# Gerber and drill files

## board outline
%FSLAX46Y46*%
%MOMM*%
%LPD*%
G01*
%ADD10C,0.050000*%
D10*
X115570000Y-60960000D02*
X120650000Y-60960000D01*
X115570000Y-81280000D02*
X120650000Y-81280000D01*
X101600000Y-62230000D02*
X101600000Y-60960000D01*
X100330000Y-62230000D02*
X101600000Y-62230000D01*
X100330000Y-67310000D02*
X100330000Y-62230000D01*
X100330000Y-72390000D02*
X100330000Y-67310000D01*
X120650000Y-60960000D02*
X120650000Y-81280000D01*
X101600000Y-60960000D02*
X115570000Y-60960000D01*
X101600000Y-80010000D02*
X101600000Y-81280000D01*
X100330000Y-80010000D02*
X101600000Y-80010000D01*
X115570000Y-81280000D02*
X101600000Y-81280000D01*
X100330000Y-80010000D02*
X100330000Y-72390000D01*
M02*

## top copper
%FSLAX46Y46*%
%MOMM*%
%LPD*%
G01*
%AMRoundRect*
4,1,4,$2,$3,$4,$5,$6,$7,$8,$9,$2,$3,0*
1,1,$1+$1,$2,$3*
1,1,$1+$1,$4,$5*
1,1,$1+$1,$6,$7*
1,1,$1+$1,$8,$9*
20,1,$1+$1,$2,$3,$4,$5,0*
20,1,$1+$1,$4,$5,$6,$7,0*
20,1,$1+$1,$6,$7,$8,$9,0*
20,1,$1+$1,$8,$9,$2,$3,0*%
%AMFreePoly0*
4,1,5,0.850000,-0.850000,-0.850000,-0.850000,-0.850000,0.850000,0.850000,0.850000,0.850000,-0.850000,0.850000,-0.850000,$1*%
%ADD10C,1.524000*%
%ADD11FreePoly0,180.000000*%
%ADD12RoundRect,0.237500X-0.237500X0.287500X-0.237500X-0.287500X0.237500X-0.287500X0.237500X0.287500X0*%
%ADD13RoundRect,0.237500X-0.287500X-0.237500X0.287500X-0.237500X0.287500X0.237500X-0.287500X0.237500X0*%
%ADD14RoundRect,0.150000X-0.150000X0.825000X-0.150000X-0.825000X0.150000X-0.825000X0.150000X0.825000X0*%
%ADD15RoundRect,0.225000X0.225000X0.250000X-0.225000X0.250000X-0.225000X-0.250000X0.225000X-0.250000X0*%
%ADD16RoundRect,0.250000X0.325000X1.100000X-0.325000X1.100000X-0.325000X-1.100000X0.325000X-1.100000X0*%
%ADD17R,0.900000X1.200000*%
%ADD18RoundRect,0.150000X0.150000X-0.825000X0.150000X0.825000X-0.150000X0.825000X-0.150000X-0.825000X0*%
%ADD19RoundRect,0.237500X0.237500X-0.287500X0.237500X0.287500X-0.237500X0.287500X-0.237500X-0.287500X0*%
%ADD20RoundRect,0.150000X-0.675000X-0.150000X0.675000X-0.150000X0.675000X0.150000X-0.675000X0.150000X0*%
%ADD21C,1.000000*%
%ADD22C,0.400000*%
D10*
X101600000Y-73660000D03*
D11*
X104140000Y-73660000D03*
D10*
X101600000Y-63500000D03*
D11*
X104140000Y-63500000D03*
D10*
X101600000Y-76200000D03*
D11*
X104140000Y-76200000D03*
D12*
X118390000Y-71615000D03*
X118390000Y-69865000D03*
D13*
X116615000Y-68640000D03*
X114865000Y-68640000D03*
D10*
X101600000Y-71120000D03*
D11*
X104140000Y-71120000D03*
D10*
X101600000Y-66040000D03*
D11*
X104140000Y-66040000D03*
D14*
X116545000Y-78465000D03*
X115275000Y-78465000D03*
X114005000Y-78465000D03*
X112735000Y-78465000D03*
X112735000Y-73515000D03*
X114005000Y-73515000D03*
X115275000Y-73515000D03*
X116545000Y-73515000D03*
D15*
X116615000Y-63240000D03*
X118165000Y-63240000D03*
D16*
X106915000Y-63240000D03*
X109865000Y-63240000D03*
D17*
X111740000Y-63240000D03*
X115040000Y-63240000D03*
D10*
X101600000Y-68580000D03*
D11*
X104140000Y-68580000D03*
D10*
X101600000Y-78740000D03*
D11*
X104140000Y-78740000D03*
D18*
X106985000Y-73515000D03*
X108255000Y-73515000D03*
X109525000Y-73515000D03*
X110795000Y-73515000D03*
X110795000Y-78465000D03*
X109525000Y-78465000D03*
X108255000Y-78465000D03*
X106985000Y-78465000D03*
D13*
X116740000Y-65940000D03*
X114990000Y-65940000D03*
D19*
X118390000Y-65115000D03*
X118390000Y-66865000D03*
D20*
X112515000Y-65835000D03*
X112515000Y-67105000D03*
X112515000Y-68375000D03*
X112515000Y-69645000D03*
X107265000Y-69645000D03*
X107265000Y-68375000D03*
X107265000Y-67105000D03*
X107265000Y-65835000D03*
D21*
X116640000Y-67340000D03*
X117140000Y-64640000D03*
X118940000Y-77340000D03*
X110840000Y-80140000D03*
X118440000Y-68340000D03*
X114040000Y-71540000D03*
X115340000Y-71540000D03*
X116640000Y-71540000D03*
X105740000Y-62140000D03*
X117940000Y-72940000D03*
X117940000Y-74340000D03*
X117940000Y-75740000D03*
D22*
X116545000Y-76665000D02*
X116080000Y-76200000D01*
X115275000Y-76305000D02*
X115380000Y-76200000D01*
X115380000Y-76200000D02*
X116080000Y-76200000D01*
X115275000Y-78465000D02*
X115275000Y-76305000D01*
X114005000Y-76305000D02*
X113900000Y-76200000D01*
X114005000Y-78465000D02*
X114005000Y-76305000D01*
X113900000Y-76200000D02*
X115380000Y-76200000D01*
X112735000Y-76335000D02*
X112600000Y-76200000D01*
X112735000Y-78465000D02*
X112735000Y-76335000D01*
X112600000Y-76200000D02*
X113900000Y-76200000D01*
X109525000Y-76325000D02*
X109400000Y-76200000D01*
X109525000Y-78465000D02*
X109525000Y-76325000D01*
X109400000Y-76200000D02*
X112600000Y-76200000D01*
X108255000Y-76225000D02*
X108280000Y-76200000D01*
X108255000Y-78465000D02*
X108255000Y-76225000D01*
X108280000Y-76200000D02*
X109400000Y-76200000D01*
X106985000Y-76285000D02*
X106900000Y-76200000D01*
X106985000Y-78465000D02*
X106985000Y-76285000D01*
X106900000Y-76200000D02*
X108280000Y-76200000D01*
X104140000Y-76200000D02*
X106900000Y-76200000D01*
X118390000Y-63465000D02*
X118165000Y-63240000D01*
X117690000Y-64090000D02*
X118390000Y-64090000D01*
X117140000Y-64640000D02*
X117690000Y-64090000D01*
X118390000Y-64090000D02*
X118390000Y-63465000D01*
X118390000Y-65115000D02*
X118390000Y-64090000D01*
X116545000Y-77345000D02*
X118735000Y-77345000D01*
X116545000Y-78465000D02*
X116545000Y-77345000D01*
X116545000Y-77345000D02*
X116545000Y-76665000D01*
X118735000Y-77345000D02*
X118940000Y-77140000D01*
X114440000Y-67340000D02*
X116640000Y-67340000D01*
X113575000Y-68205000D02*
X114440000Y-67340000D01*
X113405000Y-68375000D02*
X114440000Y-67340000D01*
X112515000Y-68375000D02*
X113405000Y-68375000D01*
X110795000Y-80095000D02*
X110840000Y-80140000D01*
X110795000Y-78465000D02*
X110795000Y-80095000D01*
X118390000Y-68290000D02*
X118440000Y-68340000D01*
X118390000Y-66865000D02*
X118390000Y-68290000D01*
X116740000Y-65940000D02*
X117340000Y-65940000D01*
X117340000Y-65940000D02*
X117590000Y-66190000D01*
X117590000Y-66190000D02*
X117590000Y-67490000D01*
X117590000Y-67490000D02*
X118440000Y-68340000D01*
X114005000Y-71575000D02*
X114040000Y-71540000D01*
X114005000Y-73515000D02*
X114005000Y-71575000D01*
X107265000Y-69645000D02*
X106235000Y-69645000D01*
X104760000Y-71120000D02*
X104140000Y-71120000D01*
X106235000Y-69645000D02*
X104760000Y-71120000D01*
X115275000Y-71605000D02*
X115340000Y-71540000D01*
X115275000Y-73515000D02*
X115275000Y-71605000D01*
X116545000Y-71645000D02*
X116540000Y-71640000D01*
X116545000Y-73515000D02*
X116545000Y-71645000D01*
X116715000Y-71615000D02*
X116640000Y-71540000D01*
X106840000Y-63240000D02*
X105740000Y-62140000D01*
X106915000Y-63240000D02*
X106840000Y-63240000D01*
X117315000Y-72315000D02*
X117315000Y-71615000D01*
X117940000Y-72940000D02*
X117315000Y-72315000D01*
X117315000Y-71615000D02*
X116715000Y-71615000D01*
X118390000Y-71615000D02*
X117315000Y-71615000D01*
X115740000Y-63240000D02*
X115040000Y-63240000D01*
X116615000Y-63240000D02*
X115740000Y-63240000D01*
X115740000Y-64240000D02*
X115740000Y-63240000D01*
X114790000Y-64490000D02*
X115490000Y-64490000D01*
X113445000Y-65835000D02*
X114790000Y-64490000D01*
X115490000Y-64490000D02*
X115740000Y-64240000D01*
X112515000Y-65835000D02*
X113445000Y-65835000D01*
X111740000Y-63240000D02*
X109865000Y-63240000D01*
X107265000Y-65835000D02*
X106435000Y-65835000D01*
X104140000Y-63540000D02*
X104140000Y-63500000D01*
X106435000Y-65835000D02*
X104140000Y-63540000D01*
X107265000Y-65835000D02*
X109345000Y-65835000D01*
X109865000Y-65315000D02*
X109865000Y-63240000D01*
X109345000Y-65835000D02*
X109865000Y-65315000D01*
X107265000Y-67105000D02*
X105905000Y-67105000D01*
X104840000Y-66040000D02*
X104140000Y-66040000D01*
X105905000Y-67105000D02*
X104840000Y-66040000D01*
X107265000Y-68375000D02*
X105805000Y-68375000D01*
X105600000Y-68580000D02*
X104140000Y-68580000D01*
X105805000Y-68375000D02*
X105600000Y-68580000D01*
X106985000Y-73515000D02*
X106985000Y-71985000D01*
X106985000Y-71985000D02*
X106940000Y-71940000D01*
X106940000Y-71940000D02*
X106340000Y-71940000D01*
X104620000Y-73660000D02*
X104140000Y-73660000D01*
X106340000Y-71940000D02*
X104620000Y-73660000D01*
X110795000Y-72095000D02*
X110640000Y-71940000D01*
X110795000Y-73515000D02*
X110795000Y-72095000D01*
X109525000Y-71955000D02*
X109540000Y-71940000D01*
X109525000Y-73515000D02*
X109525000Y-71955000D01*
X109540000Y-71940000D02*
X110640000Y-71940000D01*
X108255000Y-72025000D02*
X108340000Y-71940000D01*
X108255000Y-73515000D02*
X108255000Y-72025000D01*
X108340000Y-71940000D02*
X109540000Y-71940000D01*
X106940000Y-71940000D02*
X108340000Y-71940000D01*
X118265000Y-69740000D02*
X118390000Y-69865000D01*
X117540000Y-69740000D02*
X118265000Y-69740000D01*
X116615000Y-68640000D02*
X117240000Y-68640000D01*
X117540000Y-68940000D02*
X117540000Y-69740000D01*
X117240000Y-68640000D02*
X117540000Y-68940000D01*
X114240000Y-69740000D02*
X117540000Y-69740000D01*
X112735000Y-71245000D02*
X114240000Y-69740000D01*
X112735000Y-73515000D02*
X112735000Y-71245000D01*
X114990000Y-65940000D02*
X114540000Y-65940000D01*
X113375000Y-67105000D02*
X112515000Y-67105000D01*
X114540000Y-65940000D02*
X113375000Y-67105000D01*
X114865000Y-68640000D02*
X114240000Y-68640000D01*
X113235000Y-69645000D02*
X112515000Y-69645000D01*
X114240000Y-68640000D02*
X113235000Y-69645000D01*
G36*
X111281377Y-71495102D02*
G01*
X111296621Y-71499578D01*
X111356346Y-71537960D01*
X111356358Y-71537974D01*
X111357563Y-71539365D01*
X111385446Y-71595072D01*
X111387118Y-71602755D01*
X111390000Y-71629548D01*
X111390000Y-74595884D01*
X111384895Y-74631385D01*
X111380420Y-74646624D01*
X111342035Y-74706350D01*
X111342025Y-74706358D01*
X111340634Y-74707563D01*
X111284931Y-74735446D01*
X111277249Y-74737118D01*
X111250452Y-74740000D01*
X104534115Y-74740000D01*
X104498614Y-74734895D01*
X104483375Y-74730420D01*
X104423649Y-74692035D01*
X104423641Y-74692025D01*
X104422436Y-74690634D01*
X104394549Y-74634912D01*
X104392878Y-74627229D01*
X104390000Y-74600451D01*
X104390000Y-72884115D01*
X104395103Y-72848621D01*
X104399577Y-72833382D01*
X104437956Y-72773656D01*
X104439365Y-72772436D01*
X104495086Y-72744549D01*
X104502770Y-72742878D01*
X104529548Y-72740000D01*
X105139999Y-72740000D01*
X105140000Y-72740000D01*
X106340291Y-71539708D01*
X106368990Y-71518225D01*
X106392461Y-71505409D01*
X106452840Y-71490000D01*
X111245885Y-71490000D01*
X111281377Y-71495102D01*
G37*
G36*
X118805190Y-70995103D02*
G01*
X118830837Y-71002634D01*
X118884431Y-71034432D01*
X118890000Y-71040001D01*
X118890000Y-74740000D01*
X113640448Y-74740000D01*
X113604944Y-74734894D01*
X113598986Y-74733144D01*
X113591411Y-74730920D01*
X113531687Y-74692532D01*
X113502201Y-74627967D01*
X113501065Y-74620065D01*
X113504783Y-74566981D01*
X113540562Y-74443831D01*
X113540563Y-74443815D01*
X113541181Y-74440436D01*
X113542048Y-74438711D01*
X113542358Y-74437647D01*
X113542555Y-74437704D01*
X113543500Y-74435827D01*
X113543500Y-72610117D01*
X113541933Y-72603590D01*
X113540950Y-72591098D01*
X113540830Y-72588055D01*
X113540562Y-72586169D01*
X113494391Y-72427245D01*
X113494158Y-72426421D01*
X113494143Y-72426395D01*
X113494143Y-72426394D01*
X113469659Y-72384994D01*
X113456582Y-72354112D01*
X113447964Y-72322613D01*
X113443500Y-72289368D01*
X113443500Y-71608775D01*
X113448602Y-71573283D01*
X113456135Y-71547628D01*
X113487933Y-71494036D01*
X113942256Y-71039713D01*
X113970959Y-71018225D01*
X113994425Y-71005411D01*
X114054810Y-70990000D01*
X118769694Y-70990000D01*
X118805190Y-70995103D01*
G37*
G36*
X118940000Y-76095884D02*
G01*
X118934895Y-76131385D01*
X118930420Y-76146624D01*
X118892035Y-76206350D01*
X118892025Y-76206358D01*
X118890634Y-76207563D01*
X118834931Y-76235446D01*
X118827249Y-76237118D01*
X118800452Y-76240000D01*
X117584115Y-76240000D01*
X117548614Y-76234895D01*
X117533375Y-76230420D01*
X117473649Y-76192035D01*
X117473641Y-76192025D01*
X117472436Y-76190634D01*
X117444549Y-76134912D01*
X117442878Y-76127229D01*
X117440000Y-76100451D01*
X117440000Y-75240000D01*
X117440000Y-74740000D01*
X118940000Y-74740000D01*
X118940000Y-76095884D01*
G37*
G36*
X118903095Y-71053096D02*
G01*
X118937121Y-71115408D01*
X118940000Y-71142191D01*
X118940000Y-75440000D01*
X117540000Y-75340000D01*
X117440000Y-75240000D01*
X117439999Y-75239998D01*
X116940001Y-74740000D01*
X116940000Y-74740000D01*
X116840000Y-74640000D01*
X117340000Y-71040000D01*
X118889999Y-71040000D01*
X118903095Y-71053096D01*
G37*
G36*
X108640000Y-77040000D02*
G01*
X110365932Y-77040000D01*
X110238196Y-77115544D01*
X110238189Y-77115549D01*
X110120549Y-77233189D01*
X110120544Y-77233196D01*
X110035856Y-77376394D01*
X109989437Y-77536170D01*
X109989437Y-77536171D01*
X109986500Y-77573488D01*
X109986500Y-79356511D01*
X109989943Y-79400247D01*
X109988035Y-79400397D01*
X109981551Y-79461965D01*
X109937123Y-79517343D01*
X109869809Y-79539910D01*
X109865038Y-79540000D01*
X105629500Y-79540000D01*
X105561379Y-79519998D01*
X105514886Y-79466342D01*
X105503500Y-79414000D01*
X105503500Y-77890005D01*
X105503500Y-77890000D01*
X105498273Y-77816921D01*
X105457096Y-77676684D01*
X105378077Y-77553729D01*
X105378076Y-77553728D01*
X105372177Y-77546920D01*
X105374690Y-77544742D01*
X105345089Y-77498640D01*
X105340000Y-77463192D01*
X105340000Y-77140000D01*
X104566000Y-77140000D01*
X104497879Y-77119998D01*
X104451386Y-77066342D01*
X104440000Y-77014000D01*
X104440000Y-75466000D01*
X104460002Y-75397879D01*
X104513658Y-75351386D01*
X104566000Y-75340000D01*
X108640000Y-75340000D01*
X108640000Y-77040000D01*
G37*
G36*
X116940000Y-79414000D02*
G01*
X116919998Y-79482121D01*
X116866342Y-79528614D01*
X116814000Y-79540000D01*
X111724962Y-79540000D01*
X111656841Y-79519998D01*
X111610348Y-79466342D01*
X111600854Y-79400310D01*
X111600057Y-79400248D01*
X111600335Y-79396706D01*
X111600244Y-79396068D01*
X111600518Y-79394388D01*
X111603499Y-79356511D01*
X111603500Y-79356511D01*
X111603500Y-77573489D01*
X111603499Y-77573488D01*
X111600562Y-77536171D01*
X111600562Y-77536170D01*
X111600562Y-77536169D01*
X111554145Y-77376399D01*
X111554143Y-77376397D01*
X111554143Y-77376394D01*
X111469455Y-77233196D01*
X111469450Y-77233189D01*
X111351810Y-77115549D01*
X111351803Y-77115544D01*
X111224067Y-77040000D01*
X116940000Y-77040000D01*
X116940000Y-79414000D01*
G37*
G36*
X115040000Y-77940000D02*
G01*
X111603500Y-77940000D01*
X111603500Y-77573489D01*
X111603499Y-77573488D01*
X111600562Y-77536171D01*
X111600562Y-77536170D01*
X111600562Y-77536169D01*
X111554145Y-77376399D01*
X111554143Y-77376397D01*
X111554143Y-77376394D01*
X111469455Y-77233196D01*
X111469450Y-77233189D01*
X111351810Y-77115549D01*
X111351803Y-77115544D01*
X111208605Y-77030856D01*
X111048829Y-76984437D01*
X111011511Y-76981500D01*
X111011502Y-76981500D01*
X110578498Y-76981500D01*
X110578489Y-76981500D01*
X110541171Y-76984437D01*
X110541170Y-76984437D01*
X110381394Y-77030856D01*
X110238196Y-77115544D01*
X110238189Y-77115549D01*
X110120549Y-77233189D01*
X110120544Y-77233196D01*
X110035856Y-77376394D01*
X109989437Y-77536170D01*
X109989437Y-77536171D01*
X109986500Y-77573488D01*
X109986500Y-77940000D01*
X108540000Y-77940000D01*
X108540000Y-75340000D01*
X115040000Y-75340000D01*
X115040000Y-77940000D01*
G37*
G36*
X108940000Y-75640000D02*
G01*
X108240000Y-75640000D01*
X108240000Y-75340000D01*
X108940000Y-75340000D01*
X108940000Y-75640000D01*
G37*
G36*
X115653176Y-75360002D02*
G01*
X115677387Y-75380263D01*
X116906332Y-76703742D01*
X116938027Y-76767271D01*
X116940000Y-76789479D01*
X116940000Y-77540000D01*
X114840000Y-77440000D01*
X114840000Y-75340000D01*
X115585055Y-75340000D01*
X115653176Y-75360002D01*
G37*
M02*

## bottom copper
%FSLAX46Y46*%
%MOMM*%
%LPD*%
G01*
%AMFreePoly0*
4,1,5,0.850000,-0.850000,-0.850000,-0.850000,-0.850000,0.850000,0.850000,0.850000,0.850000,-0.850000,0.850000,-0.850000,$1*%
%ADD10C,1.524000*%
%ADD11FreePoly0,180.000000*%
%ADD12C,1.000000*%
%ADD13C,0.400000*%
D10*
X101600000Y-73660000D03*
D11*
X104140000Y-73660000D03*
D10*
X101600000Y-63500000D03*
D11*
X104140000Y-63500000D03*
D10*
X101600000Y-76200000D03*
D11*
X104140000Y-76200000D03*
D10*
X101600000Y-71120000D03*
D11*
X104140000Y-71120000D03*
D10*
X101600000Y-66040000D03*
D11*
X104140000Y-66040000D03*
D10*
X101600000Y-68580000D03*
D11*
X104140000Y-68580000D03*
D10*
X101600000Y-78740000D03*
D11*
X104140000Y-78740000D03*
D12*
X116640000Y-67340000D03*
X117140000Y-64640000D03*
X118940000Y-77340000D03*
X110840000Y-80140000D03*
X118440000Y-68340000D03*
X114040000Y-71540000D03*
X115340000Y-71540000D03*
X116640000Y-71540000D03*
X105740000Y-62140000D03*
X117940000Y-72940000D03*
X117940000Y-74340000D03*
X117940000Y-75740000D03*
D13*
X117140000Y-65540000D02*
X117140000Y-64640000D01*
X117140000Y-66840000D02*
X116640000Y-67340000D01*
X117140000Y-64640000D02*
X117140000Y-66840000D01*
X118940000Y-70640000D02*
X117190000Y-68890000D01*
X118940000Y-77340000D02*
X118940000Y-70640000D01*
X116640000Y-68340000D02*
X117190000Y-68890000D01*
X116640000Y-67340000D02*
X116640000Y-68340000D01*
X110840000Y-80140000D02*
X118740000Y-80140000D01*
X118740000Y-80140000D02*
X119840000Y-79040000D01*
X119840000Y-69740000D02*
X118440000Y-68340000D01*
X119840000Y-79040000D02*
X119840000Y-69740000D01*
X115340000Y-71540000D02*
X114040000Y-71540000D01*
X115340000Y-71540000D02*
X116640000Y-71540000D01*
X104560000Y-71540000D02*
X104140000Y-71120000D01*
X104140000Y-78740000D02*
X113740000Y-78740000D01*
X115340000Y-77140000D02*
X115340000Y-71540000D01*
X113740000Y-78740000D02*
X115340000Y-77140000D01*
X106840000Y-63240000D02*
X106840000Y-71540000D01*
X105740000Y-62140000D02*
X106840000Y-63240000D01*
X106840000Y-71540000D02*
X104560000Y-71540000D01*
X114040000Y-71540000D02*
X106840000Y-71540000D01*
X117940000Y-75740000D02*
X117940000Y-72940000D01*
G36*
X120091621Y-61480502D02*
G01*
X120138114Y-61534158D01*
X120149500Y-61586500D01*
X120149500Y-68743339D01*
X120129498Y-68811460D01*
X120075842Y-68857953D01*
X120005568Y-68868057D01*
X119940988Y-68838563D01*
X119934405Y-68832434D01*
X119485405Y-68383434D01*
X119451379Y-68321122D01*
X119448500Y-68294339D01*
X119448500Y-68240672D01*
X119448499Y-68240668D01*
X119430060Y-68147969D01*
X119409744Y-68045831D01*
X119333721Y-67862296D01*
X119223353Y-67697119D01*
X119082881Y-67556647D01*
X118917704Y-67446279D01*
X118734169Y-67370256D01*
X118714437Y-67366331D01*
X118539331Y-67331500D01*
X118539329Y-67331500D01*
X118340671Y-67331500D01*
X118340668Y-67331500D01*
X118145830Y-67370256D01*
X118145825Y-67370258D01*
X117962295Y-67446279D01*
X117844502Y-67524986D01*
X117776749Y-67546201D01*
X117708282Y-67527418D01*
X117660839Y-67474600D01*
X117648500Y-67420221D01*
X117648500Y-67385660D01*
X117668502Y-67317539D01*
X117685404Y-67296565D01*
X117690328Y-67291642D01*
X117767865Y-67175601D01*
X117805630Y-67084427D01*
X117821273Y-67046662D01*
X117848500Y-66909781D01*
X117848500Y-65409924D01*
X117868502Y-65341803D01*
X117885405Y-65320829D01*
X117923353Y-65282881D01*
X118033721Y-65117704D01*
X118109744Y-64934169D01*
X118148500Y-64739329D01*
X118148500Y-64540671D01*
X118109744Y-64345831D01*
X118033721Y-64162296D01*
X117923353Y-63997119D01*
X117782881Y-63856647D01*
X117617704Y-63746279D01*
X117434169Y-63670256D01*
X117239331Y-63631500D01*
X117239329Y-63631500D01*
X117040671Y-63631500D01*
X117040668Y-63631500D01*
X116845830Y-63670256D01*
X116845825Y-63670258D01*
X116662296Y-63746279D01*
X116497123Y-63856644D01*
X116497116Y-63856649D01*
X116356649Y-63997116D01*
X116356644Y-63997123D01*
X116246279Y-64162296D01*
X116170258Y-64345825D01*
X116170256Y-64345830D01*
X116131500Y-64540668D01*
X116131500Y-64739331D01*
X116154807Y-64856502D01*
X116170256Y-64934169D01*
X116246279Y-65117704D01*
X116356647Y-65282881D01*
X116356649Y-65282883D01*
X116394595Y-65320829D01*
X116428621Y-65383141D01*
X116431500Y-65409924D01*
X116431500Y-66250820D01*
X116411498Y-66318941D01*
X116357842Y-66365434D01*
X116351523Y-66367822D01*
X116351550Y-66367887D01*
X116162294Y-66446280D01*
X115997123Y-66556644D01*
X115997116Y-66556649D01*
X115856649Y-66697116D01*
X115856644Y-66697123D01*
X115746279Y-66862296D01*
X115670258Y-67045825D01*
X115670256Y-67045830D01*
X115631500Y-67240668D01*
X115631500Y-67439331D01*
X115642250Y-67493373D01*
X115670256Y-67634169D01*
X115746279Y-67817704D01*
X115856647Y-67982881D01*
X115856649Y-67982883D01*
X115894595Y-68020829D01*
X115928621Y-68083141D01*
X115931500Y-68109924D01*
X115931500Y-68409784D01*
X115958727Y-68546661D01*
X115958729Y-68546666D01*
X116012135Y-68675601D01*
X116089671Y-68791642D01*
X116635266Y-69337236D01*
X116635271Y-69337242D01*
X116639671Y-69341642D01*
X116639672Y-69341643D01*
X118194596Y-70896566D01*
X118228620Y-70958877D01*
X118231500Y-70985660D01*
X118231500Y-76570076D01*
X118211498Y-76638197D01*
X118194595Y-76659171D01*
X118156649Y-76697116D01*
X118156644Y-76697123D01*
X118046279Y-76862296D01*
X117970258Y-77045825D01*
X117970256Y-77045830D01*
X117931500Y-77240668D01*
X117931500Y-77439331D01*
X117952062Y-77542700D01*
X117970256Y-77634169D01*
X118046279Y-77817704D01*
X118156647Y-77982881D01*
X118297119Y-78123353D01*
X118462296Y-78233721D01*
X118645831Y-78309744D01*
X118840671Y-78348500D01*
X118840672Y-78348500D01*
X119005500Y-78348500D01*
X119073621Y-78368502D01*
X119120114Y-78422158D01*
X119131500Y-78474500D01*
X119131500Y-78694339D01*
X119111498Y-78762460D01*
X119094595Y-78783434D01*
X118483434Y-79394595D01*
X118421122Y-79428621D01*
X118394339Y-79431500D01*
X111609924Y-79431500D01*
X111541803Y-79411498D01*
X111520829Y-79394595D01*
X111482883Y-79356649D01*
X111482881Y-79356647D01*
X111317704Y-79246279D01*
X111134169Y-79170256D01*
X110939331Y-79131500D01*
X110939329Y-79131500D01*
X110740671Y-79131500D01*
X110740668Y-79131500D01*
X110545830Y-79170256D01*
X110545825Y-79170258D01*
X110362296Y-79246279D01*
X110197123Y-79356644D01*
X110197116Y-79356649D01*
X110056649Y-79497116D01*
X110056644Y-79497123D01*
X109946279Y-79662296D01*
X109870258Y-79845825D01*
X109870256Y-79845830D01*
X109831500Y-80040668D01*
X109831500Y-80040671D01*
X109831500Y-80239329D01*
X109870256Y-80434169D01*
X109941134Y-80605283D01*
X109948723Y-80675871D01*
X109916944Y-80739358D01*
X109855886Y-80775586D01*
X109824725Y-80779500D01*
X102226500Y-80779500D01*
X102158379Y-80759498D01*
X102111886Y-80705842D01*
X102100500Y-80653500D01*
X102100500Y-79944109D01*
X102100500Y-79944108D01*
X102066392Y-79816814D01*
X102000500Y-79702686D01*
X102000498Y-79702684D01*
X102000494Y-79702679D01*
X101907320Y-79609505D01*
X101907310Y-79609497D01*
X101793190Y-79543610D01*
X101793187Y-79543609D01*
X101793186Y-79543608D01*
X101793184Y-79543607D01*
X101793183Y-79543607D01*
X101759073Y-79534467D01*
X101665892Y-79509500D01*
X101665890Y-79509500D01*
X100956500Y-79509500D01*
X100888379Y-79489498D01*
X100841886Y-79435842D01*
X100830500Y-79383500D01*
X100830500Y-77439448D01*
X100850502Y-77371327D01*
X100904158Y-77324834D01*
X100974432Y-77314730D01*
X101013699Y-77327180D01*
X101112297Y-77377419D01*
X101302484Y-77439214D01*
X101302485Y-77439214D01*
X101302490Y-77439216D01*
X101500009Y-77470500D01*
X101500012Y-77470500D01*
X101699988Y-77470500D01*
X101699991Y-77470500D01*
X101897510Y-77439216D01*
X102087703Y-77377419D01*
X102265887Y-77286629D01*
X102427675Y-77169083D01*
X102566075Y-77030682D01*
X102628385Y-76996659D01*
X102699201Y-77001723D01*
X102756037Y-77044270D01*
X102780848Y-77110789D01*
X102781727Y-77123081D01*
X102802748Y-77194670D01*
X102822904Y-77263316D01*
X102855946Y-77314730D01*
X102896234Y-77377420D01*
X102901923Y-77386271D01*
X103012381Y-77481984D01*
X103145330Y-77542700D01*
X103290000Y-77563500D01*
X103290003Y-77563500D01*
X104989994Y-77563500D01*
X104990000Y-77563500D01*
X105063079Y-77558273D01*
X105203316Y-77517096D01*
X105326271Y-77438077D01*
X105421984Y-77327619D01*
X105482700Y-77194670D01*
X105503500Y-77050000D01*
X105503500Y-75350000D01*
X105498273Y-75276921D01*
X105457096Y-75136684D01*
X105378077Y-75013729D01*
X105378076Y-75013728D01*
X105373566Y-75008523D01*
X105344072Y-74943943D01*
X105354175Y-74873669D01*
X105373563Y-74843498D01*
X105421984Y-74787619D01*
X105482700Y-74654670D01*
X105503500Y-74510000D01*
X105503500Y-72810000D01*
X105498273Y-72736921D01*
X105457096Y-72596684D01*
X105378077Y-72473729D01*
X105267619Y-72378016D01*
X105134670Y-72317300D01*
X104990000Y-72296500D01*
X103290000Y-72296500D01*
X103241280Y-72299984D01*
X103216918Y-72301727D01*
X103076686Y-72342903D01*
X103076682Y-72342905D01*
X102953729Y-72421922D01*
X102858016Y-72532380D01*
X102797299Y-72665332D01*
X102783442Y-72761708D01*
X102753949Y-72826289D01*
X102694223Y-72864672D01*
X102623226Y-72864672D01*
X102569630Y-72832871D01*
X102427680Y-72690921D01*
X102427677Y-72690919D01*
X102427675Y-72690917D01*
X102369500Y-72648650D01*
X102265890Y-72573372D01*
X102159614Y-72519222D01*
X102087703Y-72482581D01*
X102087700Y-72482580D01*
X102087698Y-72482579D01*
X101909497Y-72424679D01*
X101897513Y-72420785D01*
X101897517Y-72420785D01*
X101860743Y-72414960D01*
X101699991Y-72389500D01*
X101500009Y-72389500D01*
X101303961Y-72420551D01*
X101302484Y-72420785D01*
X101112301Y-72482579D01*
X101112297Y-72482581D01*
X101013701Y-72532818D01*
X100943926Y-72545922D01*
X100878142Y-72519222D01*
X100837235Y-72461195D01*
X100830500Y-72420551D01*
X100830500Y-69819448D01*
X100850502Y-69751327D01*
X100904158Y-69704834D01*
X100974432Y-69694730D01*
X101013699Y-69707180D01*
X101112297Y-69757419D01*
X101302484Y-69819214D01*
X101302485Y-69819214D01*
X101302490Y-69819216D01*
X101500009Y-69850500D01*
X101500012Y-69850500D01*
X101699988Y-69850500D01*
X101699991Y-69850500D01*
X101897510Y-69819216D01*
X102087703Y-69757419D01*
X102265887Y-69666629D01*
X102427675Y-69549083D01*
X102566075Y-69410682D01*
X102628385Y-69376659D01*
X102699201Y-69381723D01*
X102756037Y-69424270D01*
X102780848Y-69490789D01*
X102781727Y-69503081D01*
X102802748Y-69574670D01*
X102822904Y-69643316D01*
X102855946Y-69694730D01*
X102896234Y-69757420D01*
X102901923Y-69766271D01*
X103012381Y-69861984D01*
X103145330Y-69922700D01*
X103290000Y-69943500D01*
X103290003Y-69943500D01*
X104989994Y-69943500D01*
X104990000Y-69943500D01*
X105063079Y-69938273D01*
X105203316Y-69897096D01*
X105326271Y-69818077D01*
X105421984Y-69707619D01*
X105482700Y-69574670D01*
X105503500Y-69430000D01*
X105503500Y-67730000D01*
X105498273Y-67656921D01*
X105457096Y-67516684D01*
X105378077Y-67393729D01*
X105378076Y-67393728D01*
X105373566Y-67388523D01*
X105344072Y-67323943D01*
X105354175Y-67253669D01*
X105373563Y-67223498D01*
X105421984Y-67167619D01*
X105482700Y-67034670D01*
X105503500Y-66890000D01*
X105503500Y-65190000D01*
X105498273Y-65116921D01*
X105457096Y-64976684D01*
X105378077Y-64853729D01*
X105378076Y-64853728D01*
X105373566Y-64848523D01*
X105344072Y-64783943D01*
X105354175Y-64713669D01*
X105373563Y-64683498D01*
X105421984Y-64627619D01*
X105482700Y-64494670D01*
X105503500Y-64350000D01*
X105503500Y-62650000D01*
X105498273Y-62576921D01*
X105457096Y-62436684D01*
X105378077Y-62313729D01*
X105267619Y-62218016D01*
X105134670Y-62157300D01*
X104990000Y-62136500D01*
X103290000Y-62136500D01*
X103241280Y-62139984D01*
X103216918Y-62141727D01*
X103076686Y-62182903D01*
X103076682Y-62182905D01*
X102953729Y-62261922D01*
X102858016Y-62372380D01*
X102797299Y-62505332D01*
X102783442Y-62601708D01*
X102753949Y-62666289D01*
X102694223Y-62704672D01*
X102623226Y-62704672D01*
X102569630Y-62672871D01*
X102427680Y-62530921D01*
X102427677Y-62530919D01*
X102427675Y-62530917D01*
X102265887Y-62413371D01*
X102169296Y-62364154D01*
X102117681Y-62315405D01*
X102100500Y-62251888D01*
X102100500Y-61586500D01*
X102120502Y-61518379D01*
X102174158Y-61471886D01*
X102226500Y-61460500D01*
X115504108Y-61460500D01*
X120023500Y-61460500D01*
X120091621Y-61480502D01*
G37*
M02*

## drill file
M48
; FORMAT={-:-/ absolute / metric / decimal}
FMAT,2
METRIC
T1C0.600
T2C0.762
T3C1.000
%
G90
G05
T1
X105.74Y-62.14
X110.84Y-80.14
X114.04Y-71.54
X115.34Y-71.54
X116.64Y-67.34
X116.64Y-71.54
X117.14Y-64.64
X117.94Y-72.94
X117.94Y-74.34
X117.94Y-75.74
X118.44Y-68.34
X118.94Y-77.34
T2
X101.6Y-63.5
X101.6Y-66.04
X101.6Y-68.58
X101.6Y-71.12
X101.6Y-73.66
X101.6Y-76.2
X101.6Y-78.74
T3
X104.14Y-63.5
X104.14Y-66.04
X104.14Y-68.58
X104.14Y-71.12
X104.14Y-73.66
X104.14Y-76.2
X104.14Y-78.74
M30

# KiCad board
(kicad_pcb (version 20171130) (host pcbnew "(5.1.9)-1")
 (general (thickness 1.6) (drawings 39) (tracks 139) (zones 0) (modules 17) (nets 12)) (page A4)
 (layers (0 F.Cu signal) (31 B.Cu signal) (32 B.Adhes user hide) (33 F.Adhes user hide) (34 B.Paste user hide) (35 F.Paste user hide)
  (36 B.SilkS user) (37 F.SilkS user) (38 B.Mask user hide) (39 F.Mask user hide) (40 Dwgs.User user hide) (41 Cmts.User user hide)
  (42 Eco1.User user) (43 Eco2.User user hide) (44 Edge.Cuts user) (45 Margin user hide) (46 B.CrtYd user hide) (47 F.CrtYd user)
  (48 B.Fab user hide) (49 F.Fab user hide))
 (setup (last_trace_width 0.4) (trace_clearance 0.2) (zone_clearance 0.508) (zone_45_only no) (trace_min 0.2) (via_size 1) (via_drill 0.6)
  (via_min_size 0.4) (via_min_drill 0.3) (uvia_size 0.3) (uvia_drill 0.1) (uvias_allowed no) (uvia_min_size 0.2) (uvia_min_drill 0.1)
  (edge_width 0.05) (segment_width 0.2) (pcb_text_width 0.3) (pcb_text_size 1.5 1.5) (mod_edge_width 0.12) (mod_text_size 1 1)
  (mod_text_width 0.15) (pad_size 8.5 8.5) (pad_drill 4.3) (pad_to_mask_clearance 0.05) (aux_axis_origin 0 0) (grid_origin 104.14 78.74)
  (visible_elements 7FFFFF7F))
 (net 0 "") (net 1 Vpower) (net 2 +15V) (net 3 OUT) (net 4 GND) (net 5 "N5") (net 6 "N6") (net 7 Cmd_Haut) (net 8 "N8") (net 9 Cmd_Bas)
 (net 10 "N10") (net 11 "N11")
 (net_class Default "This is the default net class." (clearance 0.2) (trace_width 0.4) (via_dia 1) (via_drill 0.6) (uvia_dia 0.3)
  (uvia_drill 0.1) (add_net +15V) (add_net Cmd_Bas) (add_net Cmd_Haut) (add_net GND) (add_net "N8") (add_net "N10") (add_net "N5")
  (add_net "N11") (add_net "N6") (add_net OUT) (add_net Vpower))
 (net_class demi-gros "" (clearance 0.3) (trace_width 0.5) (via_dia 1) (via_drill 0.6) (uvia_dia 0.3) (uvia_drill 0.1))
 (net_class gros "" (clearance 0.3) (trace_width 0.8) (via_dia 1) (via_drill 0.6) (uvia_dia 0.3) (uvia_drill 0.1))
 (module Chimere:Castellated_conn (layer F.Cu) (at 104.14 73.66 180)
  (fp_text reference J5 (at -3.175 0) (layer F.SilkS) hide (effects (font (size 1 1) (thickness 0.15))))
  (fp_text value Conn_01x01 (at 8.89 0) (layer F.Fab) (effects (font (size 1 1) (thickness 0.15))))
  (pad 1 thru_hole circle (at 2.54 0 180) (size 1.524 1.524) (drill 0.762) (layers *.Cu *.Mask) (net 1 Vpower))
  (pad 1 thru_hole custom (at 0 0 180) (size 1.7 1.7) (drill 1) (layers *.Cu *.Mask) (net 1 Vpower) (zone_connect 2)
   (options (clearance outline) (anchor rect)) (primitives)))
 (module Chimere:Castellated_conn (layer F.Cu) (at 104.14 63.5 180)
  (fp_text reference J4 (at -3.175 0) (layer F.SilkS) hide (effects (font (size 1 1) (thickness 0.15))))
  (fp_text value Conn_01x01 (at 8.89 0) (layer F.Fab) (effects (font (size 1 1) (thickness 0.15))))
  (pad 1 thru_hole circle (at 2.54 0 180) (size 1.524 1.524) (drill 0.762) (layers *.Cu *.Mask) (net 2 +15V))
  (pad 1 thru_hole custom (at 0 0 180) (size 1.7 1.7) (drill 1) (layers *.Cu *.Mask) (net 2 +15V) (zone_connect 2)
   (options (clearance outline) (anchor rect)) (primitives)))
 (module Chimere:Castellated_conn (layer F.Cu) (at 104.14 76.2 180)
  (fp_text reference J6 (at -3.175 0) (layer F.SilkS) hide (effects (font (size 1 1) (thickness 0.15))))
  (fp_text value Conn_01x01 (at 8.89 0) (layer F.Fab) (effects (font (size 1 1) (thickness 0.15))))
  (pad 1 thru_hole circle (at 2.54 0 180) (size 1.524 1.524) (drill 0.762) (layers *.Cu *.Mask) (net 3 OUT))
  (pad 1 thru_hole custom (at 0 0 180) (size 1.7 1.7) (drill 1) (layers *.Cu *.Mask) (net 3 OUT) (zone_connect 2)
   (options (clearance outline) (anchor rect)) (primitives)))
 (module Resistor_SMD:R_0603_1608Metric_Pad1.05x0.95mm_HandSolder (layer F.Cu) (at 118.39 70.74 270)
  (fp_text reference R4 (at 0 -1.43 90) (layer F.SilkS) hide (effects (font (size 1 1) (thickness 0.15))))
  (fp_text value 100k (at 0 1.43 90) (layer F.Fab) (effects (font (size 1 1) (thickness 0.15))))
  (pad 2 smd roundrect (at 0.875 0 270) (size 1.05 0.95) (layers F.Cu F.Paste F.Mask) (roundrect_rratio 0.25) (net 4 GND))
  (pad 1 smd roundrect (at -0.875 0 270) (size 1.05 0.95) (layers F.Cu F.Paste F.Mask) (roundrect_rratio 0.25) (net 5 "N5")))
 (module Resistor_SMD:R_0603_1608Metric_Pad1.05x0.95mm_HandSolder (layer F.Cu) (at 115.74 68.64)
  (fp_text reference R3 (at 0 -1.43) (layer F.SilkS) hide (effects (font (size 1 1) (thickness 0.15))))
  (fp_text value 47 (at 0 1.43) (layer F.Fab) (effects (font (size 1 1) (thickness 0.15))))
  (pad 2 smd roundrect (at 0.875 0) (size 1.05 0.95) (layers F.Cu F.Paste F.Mask) (roundrect_rratio 0.25) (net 5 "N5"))
  (pad 1 smd roundrect (at -0.875 0) (size 1.05 0.95) (layers F.Cu F.Paste F.Mask) (roundrect_rratio 0.25) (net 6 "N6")))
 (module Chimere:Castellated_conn (layer F.Cu) (at 104.14 71.12 180)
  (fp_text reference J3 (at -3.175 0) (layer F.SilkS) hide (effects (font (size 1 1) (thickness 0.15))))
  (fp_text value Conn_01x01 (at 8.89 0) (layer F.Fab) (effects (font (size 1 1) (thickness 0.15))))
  (pad 1 thru_hole circle (at 2.54 0 180) (size 1.524 1.524) (drill 0.762) (layers *.Cu *.Mask) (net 4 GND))
  (pad 1 thru_hole custom (at 0 0 180) (size 1.7 1.7) (drill 1) (layers *.Cu *.Mask) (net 4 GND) (zone_connect 2)
   (options (clearance outline) (anchor rect)) (primitives)))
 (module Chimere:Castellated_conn (layer F.Cu) (at 104.14 66.04 180)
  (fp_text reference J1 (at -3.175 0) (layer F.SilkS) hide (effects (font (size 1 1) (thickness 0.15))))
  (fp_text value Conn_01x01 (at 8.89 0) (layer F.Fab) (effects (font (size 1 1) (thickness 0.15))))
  (pad 1 thru_hole circle (at 2.54 0 180) (size 1.524 1.524) (drill 0.762) (layers *.Cu *.Mask) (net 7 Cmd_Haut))
  (pad 1 thru_hole custom (at 0 0 180) (size 1.7 1.7) (drill 1) (layers *.Cu *.Mask) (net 7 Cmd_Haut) (zone_connect 2)
   (options (clearance outline) (anchor rect)) (primitives)))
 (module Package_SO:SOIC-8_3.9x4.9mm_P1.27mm (layer F.Cu) (at 114.64 75.99 270)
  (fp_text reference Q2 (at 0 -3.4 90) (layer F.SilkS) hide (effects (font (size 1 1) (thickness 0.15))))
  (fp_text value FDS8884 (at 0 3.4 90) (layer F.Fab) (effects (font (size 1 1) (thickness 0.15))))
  (pad 8 smd roundrect (at 2.475 -1.905 270) (size 1.95 0.6) (layers F.Cu F.Paste F.Mask) (roundrect_rratio 0.25) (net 3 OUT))
  (pad 7 smd roundrect (at 2.475 -0.635 270) (size 1.95 0.6) (layers F.Cu F.Paste F.Mask) (roundrect_rratio 0.25) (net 3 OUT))
  (pad 6 smd roundrect (at 2.475 0.635 270) (size 1.95 0.6) (layers F.Cu F.Paste F.Mask) (roundrect_rratio 0.25) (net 3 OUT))
  (pad 5 smd roundrect (at 2.475 1.905 270) (size 1.95 0.6) (layers F.Cu F.Paste F.Mask) (roundrect_rratio 0.25) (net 3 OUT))
  (pad 4 smd roundrect (at -2.475 1.905 270) (size 1.95 0.6) (layers F.Cu F.Paste F.Mask) (roundrect_rratio 0.25) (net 5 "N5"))
  (pad 3 smd roundrect (at -2.475 0.635 270) (size 1.95 0.6) (layers F.Cu F.Paste F.Mask) (roundrect_rratio 0.25) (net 4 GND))
  (pad 2 smd roundrect (at -2.475 -0.635 270) (size 1.95 0.6) (layers F.Cu F.Paste F.Mask) (roundrect_rratio 0.25) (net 4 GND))
  (pad 1 smd roundrect (at -2.475 -1.905 270) (size 1.95 0.6) (layers F.Cu F.Paste F.Mask) (roundrect_rratio 0.25) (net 4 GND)))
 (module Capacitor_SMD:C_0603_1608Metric (layer F.Cu) (at 117.39 63.24 180)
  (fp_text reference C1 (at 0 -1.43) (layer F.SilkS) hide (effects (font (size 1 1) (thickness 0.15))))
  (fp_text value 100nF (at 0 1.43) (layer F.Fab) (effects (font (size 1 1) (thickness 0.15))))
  (pad 2 smd roundrect (at 0.775 0 180) (size 0.9 0.95) (layers F.Cu F.Paste F.Mask) (roundrect_rratio 0.25) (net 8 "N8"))
  (pad 1 smd roundrect (at -0.775 0 180) (size 0.9 0.95) (layers F.Cu F.Paste F.Mask) (roundrect_rratio 0.25) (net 3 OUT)))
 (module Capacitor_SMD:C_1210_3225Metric (layer F.Cu) (at 108.39 63.24 180)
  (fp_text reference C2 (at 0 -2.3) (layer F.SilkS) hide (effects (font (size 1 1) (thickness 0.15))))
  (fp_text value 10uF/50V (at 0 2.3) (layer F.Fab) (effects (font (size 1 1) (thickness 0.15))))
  (pad 2 smd roundrect (at 1.475 0 180) (size 1.15 2.7) (layers F.Cu F.Paste F.Mask) (roundrect_rratio 0.217391) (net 4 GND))
  (pad 1 smd roundrect (at -1.475 0 180) (size 1.15 2.7) (layers F.Cu F.Paste F.Mask) (roundrect_rratio 0.217391) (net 2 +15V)))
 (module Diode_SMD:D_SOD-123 (layer F.Cu) (at 113.39 63.24 180)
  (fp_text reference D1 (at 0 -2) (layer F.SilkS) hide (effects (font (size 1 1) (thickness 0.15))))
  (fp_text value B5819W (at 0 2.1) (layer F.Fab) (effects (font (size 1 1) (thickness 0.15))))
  (pad 2 smd rect (at 1.65 0 180) (size 0.9 1.2) (layers F.Cu F.Paste F.Mask) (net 2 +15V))
  (pad 1 smd rect (at -1.65 0 180) (size 0.9 1.2) (layers F.Cu F.Paste F.Mask) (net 8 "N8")))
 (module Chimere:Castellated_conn (layer F.Cu) (at 104.14 68.58 180)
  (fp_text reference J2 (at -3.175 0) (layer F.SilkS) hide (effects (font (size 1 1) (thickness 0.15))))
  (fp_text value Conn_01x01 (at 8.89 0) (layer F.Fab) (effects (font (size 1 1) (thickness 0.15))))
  (pad 1 thru_hole circle (at 2.54 0 180) (size 1.524 1.524) (drill 0.762) (layers *.Cu *.Mask) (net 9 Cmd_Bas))
  (pad 1 thru_hole custom (at 0 0 180) (size 1.7 1.7) (drill 1) (layers *.Cu *.Mask) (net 9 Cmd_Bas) (zone_connect 2)
   (options (clearance outline) (anchor rect)) (primitives)))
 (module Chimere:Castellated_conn (layer F.Cu) (at 104.14 78.74 180)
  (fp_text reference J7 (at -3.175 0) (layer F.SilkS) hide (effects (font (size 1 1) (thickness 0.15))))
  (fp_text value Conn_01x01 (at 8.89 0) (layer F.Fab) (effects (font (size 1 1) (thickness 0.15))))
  (pad 1 thru_hole circle (at 2.54 0 180) (size 1.524 1.524) (drill 0.762) (layers *.Cu *.Mask) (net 4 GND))
  (pad 1 thru_hole custom (at 0 0 180) (size 1.7 1.7) (drill 1) (layers *.Cu *.Mask) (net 4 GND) (zone_connect 2)
   (options (clearance outline) (anchor rect)) (primitives)))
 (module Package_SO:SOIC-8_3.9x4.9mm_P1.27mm (layer F.Cu) (at 108.89 75.99 90)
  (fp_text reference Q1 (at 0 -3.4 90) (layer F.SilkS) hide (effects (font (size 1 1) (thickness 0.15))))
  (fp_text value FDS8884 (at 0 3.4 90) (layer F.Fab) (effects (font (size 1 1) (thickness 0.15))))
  (pad 8 smd roundrect (at 2.475 -1.905 90) (size 1.95 0.6) (layers F.Cu F.Paste F.Mask) (roundrect_rratio 0.25) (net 1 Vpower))
  (pad 7 smd roundrect (at 2.475 -0.635 90) (size 1.95 0.6) (layers F.Cu F.Paste F.Mask) (roundrect_rratio 0.25) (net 1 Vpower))
  (pad 6 smd roundrect (at 2.475 0.635 90) (size 1.95 0.6) (layers F.Cu F.Paste F.Mask) (roundrect_rratio 0.25) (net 1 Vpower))
  (pad 5 smd roundrect (at 2.475 1.905 90) (size 1.95 0.6) (layers F.Cu F.Paste F.Mask) (roundrect_rratio 0.25) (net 1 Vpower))
  (pad 4 smd roundrect (at -2.475 1.905 90) (size 1.95 0.6) (layers F.Cu F.Paste F.Mask) (roundrect_rratio 0.25) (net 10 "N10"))
  (pad 3 smd roundrect (at -2.475 0.635 90) (size 1.95 0.6) (layers F.Cu F.Paste F.Mask) (roundrect_rratio 0.25) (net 3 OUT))
  (pad 2 smd roundrect (at -2.475 -0.635 90) (size 1.95 0.6) (layers F.Cu F.Paste F.Mask) (roundrect_rratio 0.25) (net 3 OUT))
  (pad 1 smd roundrect (at -2.475 -1.905 90) (size 1.95 0.6) (layers F.Cu F.Paste F.Mask) (roundrect_rratio 0.25) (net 3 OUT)))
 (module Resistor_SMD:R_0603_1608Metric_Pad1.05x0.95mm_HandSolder (layer F.Cu) (at 115.865 65.94)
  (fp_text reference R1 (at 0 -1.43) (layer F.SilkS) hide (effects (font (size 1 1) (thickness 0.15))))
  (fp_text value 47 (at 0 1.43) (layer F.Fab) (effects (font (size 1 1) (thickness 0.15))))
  (pad 2 smd roundrect (at 0.875 0) (size 1.05 0.95) (layers F.Cu F.Paste F.Mask) (roundrect_rratio 0.25) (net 10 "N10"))
  (pad 1 smd roundrect (at -0.875 0) (size 1.05 0.95) (layers F.Cu F.Paste F.Mask) (roundrect_rratio 0.25) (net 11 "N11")))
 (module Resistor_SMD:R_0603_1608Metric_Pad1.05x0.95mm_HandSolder (layer F.Cu) (at 118.39 65.99 90)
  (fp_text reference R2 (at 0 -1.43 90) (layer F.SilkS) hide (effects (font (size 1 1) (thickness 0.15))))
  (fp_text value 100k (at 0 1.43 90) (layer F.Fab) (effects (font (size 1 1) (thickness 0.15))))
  (pad 2 smd roundrect (at 0.875 0 90) (size 1.05 0.95) (layers F.Cu F.Paste F.Mask) (roundrect_rratio 0.25) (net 3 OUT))
  (pad 1 smd roundrect (at -0.875 0 90) (size 1.05 0.95) (layers F.Cu F.Paste F.Mask) (roundrect_rratio 0.25) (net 10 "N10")))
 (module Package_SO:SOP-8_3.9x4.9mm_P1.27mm (layer F.Cu) (at 109.89 67.74)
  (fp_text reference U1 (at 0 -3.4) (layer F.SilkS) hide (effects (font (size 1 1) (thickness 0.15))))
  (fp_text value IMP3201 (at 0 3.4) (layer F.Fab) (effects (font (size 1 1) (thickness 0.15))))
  (pad 8 smd roundrect (at 2.625 -1.905) (size 1.65 0.6) (layers F.Cu F.Paste F.Mask) (roundrect_rratio 0.25) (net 8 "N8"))
  (pad 7 smd roundrect (at 2.625 -0.635) (size 1.65 0.6) (layers F.Cu F.Paste F.Mask) (roundrect_rratio 0.25) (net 11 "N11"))
  (pad 6 smd roundrect (at 2.625 0.635) (size 1.65 0.6) (layers F.Cu F.Paste F.Mask) (roundrect_rratio 0.25) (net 3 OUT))
  (pad 5 smd roundrect (at 2.625 1.905) (size 1.65 0.6) (layers F.Cu F.Paste F.Mask) (roundrect_rratio 0.25) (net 6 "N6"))
  (pad 4 smd roundrect (at -2.625 1.905) (size 1.65 0.6) (layers F.Cu F.Paste F.Mask) (roundrect_rratio 0.25) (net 4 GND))
  (pad 3 smd roundrect (at -2.625 0.635) (size 1.65 0.6) (layers F.Cu F.Paste F.Mask) (roundrect_rratio 0.25) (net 9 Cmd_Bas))
  (pad 2 smd roundrect (at -2.625 -0.635) (size 1.65 0.6) (layers F.Cu F.Paste F.Mask) (roundrect_rratio 0.25) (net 7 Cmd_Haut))
  (pad 1 smd roundrect (at -2.625 -1.905) (size 1.65 0.6) (layers F.Cu F.Paste F.Mask) (roundrect_rratio 0.25) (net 2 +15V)))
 (gr_line (start 115.57 60.96) (end 120.65 60.96) (layer Edge.Cuts) (width 0.05))
 (gr_line (start 115.57 81.28) (end 120.65 81.28) (layer Edge.Cuts) (width 0.05))
 (gr_line (start 101.6 62.23) (end 101.6 60.96) (layer Edge.Cuts) (width 0.05))
 (gr_line (start 100.33 62.23) (end 101.6 62.23) (layer Edge.Cuts) (width 0.05))
 (gr_line (start 100.33 67.31) (end 100.33 62.23) (layer Edge.Cuts) (width 0.05))
 (gr_line (start 100.33 72.39) (end 100.33 67.31) (layer Edge.Cuts) (width 0.05))
 (gr_line (start 120.65 60.96) (end 120.65 81.28) (layer Edge.Cuts) (width 0.05))
 (gr_line (start 101.6 60.96) (end 115.57 60.96) (layer Edge.Cuts) (width 0.05))
 (gr_line (start 101.6 80.01) (end 101.6 81.28) (layer Edge.Cuts) (width 0.05))
 (gr_line (start 100.33 80.01) (end 101.6 80.01) (layer Edge.Cuts) (width 0.05))
 (gr_line (start 115.57 81.28) (end 101.6 81.28) (layer Edge.Cuts) (width 0.05))
 (gr_line (start 100.33 80.01) (end 100.33 72.39) (layer Edge.Cuts) (width 0.05))
 (segment (start 116.545 76.665) (end 116.08 76.2) (width 0.4) (layer F.Cu) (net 3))
 (segment (start 115.275 76.305) (end 115.38 76.2) (width 0.4) (layer F.Cu) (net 3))
 (segment (start 115.38 76.2) (end 116.08 76.2) (width 0.4) (layer F.Cu) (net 3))
 (segment (start 115.275 78.465) (end 115.275 76.305) (width 0.4) (layer F.Cu) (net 3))
 (segment (start 114.005 76.305) (end 113.9 76.2) (width 0.4) (layer F.Cu) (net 3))
 (segment (start 114.005 78.465) (end 114.005 76.305) (width 0.4) (layer F.Cu) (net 3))
 (segment (start 113.9 76.2) (end 115.38 76.2) (width 0.4) (layer F.Cu) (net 3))
 (segment (start 112.735 76.335) (end 112.6 76.2) (width 0.4) (layer F.Cu) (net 3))
 (segment (start 112.735 78.465) (end 112.735 76.335) (width 0.4) (layer F.Cu) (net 3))
 (segment (start 112.6 76.2) (end 113.9 76.2) (width 0.4) (layer F.Cu) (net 3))
 (segment (start 109.525 76.325) (end 109.4 76.2) (width 0.4) (layer F.Cu) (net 3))
 (segment (start 109.525 78.465) (end 109.525 76.325) (width 0.4) (layer F.Cu) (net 3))
 (segment (start 109.4 76.2) (end 112.6 76.2) (width 0.4) (layer F.Cu) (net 3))
 (segment (start 108.255 76.225) (end 108.28 76.2) (width 0.4) (layer F.Cu) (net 3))
 (segment (start 108.255 78.465) (end 108.255 76.225) (width 0.4) (layer F.Cu) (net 3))
 (segment (start 108.28 76.2) (end 109.4 76.2) (width 0.4) (layer F.Cu) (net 3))
 (segment (start 106.985 76.285) (end 106.9 76.2) (width 0.4) (layer F.Cu) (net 3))
 (segment (start 106.985 78.465) (end 106.985 76.285) (width 0.4) (layer F.Cu) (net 3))
 (segment (start 106.9 76.2) (end 108.28 76.2) (width 0.4) (layer F.Cu) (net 3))
 (segment (start 104.14 76.2) (end 106.9 76.2) (width 0.4) (layer F.Cu) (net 3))
 (segment (start 118.39 63.465) (end 118.165 63.24) (width 0.4) (layer F.Cu) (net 3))
 (via (at 116.64 67.34) (size 1) (drill 0.6) (layers F.Cu B.Cu) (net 3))
 (via (at 117.14 64.64) (size 1) (drill 0.6) (layers F.Cu B.Cu) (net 3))
 (segment (start 117.14 65.54) (end 117.14 64.64) (width 0.4) (layer B.Cu) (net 3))
 (segment (start 117.69 64.09) (end 118.39 64.09) (width 0.4) (layer F.Cu) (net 3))
 (segment (start 117.14 64.64) (end 117.69 64.09) (width 0.4) (layer F.Cu) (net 3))
 (segment (start 118.39 64.09) (end 118.39 63.465) (width 0.4) (layer F.Cu) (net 3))
 (segment (start 118.39 65.115) (end 118.39 64.09) (width 0.4) (layer F.Cu) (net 3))
 (via (at 118.94 77.34) (size 1) (drill 0.6) (layers F.Cu B.Cu) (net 3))
 (segment (start 116.545 77.345) (end 118.735 77.345) (width 0.4) (layer F.Cu) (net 3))
 (segment (start 116.545 78.465) (end 116.545 77.345) (width 0.4) (layer F.Cu) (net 3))
 (segment (start 116.545 77.345) (end 116.545 76.665) (width 0.4) (layer F.Cu) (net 3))
 (segment (start 118.735 77.345) (end 118.94 77.14) (width 0.4) (layer F.Cu) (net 3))
 (segment (start 117.14 66.84) (end 116.64 67.34) (width 0.4) (layer B.Cu) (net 3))
 (segment (start 117.14 64.64) (end 117.14 66.84) (width 0.4) (layer B.Cu) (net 3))
 (segment (start 118.94 70.64) (end 117.19 68.89) (width 0.4) (layer B.Cu) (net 3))
 (segment (start 118.94 77.34) (end 118.94 70.64) (width 0.4) (layer B.Cu) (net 3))
 (segment (start 116.64 68.34) (end 117.19 68.89) (width 0.4) (layer B.Cu) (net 3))
 (segment (start 116.64 67.34) (end 116.64 68.34) (width 0.4) (layer B.Cu) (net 3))
 (segment (start 114.44 67.34) (end 116.64 67.34) (width 0.4) (layer F.Cu) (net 3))
 (segment (start 113.575 68.205) (end 114.44 67.34) (width 0.4) (layer F.Cu) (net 3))
 (segment (start 113.405 68.375) (end 114.44 67.34) (width 0.4) (layer F.Cu) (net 3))
 (segment (start 112.515 68.375) (end 113.405 68.375) (width 0.4) (layer F.Cu) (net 3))
 (via (at 110.84 80.14) (size 1) (drill 0.6) (layers F.Cu B.Cu) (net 10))
 (segment (start 110.795 80.095) (end 110.84 80.14) (width 0.4) (layer F.Cu) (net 10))
 (segment (start 110.795 78.465) (end 110.795 80.095) (width 0.4) (layer F.Cu) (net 10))
 (segment (start 110.84 80.14) (end 118.74 80.14) (width 0.4) (layer B.Cu) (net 10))
 (segment (start 118.74 80.14) (end 119.84 79.04) (width 0.4) (layer B.Cu) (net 10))
 (via (at 118.44 68.34) (size 1) (drill 0.6) (layers F.Cu B.Cu) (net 10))
 (segment (start 119.84 69.74) (end 118.44 68.34) (width 0.4) (layer B.Cu) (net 10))
 (segment (start 119.84 79.04) (end 119.84 69.74) (width 0.4) (layer B.Cu) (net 10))
 (segment (start 118.39 68.29) (end 118.44 68.34) (width 0.4) (layer F.Cu) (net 10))
 (segment (start 118.39 66.865) (end 118.39 68.29) (width 0.4) (layer F.Cu) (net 10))
 (segment (start 116.74 65.94) (end 117.34 65.94) (width 0.4) (layer F.Cu) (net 10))
 (segment (start 117.34 65.94) (end 117.59 66.19) (width 0.4) (layer F.Cu) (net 10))
 (segment (start 117.59 66.19) (end 117.59 67.49) (width 0.4) (layer F.Cu) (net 10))
 (segment (start 117.59 67.49) (end 118.44 68.34) (width 0.4) (layer F.Cu) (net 10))
 (via (at 114.04 71.54) (size 1) (drill 0.6) (layers F.Cu B.Cu) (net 4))
 (segment (start 114.005 71.575) (end 114.04 71.54) (width 0.4) (layer F.Cu) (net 4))
 (segment (start 114.005 73.515) (end 114.005 71.575) (width 0.4) (layer F.Cu) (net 4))
 (segment (start 107.265 69.645) (end 106.235 69.645) (width 0.4) (layer F.Cu) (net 4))
 (segment (start 104.76 71.12) (end 104.14 71.12) (width 0.4) (layer F.Cu) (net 4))
 (segment (start 106.235 69.645) (end 104.76 71.12) (width 0.4) (layer F.Cu) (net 4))
 (via (at 115.34 71.54) (size 1) (drill 0.6) (layers F.Cu B.Cu) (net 4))
 (segment (start 115.275 71.605) (end 115.34 71.54) (width 0.4) (layer F.Cu) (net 4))
 (segment (start 115.275 73.515) (end 115.275 71.605) (width 0.4) (layer F.Cu) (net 4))
 (segment (start 115.34 71.54) (end 114.04 71.54) (width 0.4) (layer B.Cu) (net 4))
 (via (at 116.64 71.54) (size 1) (drill 0.6) (layers F.Cu B.Cu) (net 4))
 (segment (start 116.545 71.645) (end 116.54 71.64) (width 0.4) (layer F.Cu) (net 4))
 (segment (start 116.545 73.515) (end 116.545 71.645) (width 0.4) (layer F.Cu) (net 4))
 (segment (start 115.34 71.54) (end 116.64 71.54) (width 0.4) (layer B.Cu) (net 4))
 (segment (start 116.715 71.615) (end 116.64 71.54) (width 0.4) (layer F.Cu) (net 4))
 (segment (start 104.56 71.54) (end 104.14 71.12) (width 0.4) (layer B.Cu) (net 4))
 (segment (start 104.14 78.74) (end 113.74 78.74) (width 0.4) (layer B.Cu) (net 4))
 (segment (start 115.34 77.14) (end 115.34 71.54) (width 0.4) (layer B.Cu) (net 4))
 (segment (start 113.74 78.74) (end 115.34 77.14) (width 0.4) (layer B.Cu) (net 4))
 (via (at 105.74 62.14) (size 1) (drill 0.6) (layers F.Cu B.Cu) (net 4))
 (segment (start 106.84 63.24) (end 105.74 62.14) (width 0.4) (layer F.Cu) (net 4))
 (segment (start 106.915 63.24) (end 106.84 63.24) (width 0.4) (layer F.Cu) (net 4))
 (segment (start 106.84 63.24) (end 106.84 71.54) (width 0.4) (layer B.Cu) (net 4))
 (segment (start 105.74 62.14) (end 106.84 63.24) (width 0.4) (layer B.Cu) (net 4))
 (segment (start 106.84 71.54) (end 104.56 71.54) (width 0.4) (layer B.Cu) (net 4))
 (segment (start 114.04 71.54) (end 106.84 71.54) (width 0.4) (layer B.Cu) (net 4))
 (via (at 117.94 72.94) (size 1) (drill 0.6) (layers F.Cu B.Cu) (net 4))
 (via (at 117.94 74.34) (size 1) (drill 0.6) (layers F.Cu B.Cu) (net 4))
 (via (at 117.94 75.74) (size 1) (drill 0.6) (layers F.Cu B.Cu) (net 4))
 (segment (start 117.94 75.74) (end 117.94 72.94) (width 0.4) (layer B.Cu) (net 4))
 (segment (start 117.315 72.315) (end 117.315 71.615) (width 0.4) (layer F.Cu) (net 4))
 (segment (start 117.94 72.94) (end 117.315 72.315) (width 0.4) (layer F.Cu) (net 4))
 (segment (start 117.315 71.615) (end 116.715 71.615) (width 0.4) (layer F.Cu) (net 4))
 (segment (start 118.39 71.615) (end 117.315 71.615) (width 0.4) (layer F.Cu) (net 4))
 (segment (start 115.74 63.24) (end 115.04 63.24) (width 0.4) (layer F.Cu) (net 8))
 (segment (start 116.615 63.24) (end 115.74 63.24) (width 0.4) (layer F.Cu) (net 8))
 (segment (start 115.74 64.24) (end 115.74 63.24) (width 0.4) (layer F.Cu) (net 8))
 (segment (start 114.79 64.49) (end 115.49 64.49) (width 0.4) (layer F.Cu) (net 8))
 (segment (start 113.445 65.835) (end 114.79 64.49) (width 0.4) (layer F.Cu) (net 8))
 (segment (start 115.49 64.49) (end 115.74 64.24) (width 0.4) (layer F.Cu) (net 8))
 (segment (start 112.515 65.835) (end 113.445 65.835) (width 0.4) (layer F.Cu) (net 8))
 (segment (start 111.74 63.24) (end 109.865 63.24) (width 0.4) (layer F.Cu) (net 2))
 (segment (start 107.265 65.835) (end 106.435 65.835) (width 0.4) (layer F.Cu) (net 2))
 (segment (start 104.14 63.54) (end 104.14 63.5) (width 0.4) (layer F.Cu) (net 2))
 (segment (start 106.435 65.835) (end 104.14 63.54) (width 0.4) (layer F.Cu) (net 2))
 (segment (start 107.265 65.835) (end 109.345 65.835) (width 0.4) (layer F.Cu) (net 2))
 (segment (start 109.865 65.315) (end 109.865 63.24) (width 0.4) (layer F.Cu) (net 2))
 (segment (start 109.345 65.835) (end 109.865 65.315) (width 0.4) (layer F.Cu) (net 2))
 (segment (start 107.265 67.105) (end 105.905 67.105) (width 0.4) (layer F.Cu) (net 7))
 (segment (start 104.84 66.04) (end 104.14 66.04) (width 0.4) (layer F.Cu) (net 7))
 (segment (start 105.905 67.105) (end 104.84 66.04) (width 0.4) (layer F.Cu) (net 7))
 (segment (start 107.265 68.375) (end 105.805 68.375) (width 0.4) (layer F.Cu) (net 9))
 (segment (start 105.6 68.58) (end 104.14 68.58) (width 0.4) (layer F.Cu) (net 9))
 (segment (start 105.805 68.375) (end 105.6 68.58) (width 0.4) (layer F.Cu) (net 9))
 (segment (start 106.985 73.515) (end 106.985 71.985) (width 0.4) (layer F.Cu) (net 1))
 (segment (start 106.985 71.985) (end 106.94 71.94) (width 0.4) (layer F.Cu) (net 1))
 (segment (start 106.94 71.94) (end 106.34 71.94) (width 0.4) (layer F.Cu) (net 1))
 (segment (start 104.62 73.66) (end 104.14 73.66) (width 0.4) (layer F.Cu) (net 1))
 (segment (start 106.34 71.94) (end 104.62 73.66) (width 0.4) (layer F.Cu) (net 1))
 (segment (start 110.795 72.095) (end 110.64 71.94) (width 0.4) (layer F.Cu) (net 1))
 (segment (start 110.795 73.515) (end 110.795 72.095) (width 0.4) (layer F.Cu) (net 1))
 (segment (start 109.525 71.955) (end 109.54 71.94) (width 0.4) (layer F.Cu) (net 1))
 (segment (start 109.525 73.515) (end 109.525 71.955) (width 0.4) (layer F.Cu) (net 1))
 (segment (start 109.54 71.94) (end 110.64 71.94) (width 0.4) (layer F.Cu) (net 1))
 (segment (start 108.255 72.025) (end 108.34 71.94) (width 0.4) (layer F.Cu) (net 1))
 (segment (start 108.255 73.515) (end 108.255 72.025) (width 0.4) (layer F.Cu) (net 1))
 (segment (start 108.34 71.94) (end 109.54 71.94) (width 0.4) (layer F.Cu) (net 1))
 (segment (start 106.94 71.94) (end 108.34 71.94) (width 0.4) (layer F.Cu) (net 1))
 (segment (start 118.265 69.74) (end 118.39 69.865) (width 0.4) (layer F.Cu) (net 5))
 (segment (start 117.54 69.74) (end 118.265 69.74) (width 0.4) (layer F.Cu) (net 5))
 (segment (start 116.615 68.64) (end 117.24 68.64) (width 0.4) (layer F.Cu) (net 5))
 (segment (start 117.54 68.94) (end 117.54 69.74) (width 0.4) (layer F.Cu) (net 5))
 (segment (start 117.24 68.64) (end 117.54 68.94) (width 0.4) (layer F.Cu) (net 5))
 (segment (start 114.24 69.74) (end 117.54 69.74) (width 0.4) (layer F.Cu) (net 5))
 (segment (start 112.735 71.245) (end 114.24 69.74) (width 0.4) (layer F.Cu) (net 5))
 (segment (start 112.735 73.515) (end 112.735 71.245) (width 0.4) (layer F.Cu) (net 5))
 (segment (start 114.99 65.94) (end 114.54 65.94) (width 0.4) (layer F.Cu) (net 11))
 (segment (start 113.375 67.105) (end 112.515 67.105) (width 0.4) (layer F.Cu) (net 11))
 (segment (start 114.54 65.94) (end 113.375 67.105) (width 0.4) (layer F.Cu) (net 11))
 (segment (start 114.865 68.64) (end 114.24 68.64) (width 0.4) (layer F.Cu) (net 6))
 (segment (start 113.235 69.645) (end 112.515 69.645) (width 0.4) (layer F.Cu) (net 6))
 (segment (start 114.24 68.64) (end 113.235 69.645) (width 0.4) (layer F.Cu) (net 6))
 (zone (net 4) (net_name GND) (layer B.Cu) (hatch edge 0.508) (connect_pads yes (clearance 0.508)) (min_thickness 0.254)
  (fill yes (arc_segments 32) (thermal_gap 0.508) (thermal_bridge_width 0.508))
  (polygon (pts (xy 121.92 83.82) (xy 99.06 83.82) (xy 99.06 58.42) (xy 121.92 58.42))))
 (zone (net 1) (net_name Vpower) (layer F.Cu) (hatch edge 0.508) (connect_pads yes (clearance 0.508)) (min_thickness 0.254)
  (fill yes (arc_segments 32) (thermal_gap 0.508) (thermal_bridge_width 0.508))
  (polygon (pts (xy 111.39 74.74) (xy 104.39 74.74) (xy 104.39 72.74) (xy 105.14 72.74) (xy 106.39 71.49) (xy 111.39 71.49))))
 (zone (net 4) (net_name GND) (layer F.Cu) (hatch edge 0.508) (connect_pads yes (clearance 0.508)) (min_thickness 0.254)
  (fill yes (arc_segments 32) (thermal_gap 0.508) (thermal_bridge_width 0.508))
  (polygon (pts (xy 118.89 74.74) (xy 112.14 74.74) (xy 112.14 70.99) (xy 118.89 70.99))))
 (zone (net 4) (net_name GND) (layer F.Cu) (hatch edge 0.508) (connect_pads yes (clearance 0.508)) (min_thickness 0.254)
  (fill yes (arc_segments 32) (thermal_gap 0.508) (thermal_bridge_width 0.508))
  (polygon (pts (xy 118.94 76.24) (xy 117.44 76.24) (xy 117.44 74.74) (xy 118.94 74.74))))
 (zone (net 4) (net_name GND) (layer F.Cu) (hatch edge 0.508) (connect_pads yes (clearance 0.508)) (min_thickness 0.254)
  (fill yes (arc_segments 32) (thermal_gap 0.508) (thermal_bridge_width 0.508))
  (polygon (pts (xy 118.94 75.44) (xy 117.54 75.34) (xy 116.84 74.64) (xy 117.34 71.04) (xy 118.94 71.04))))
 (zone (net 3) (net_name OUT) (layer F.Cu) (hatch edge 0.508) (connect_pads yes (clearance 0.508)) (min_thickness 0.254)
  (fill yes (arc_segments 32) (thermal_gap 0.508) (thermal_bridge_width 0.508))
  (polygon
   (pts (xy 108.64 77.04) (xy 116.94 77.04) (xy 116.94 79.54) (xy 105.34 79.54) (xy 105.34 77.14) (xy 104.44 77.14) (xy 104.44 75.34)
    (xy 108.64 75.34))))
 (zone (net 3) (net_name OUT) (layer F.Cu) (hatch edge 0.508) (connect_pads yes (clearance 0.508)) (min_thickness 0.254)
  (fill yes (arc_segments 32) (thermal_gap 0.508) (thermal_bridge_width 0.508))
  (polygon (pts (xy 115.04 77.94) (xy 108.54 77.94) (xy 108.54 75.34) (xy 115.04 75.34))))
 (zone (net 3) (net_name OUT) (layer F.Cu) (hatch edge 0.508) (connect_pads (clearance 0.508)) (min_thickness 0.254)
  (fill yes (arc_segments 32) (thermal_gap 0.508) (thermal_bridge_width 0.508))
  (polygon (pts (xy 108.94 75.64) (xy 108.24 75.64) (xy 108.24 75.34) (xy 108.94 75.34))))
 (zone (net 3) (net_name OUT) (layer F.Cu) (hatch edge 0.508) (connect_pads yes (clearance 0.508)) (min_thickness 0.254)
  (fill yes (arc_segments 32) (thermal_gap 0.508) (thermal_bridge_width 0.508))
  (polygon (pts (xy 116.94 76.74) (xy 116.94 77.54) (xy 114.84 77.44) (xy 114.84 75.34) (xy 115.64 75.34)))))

